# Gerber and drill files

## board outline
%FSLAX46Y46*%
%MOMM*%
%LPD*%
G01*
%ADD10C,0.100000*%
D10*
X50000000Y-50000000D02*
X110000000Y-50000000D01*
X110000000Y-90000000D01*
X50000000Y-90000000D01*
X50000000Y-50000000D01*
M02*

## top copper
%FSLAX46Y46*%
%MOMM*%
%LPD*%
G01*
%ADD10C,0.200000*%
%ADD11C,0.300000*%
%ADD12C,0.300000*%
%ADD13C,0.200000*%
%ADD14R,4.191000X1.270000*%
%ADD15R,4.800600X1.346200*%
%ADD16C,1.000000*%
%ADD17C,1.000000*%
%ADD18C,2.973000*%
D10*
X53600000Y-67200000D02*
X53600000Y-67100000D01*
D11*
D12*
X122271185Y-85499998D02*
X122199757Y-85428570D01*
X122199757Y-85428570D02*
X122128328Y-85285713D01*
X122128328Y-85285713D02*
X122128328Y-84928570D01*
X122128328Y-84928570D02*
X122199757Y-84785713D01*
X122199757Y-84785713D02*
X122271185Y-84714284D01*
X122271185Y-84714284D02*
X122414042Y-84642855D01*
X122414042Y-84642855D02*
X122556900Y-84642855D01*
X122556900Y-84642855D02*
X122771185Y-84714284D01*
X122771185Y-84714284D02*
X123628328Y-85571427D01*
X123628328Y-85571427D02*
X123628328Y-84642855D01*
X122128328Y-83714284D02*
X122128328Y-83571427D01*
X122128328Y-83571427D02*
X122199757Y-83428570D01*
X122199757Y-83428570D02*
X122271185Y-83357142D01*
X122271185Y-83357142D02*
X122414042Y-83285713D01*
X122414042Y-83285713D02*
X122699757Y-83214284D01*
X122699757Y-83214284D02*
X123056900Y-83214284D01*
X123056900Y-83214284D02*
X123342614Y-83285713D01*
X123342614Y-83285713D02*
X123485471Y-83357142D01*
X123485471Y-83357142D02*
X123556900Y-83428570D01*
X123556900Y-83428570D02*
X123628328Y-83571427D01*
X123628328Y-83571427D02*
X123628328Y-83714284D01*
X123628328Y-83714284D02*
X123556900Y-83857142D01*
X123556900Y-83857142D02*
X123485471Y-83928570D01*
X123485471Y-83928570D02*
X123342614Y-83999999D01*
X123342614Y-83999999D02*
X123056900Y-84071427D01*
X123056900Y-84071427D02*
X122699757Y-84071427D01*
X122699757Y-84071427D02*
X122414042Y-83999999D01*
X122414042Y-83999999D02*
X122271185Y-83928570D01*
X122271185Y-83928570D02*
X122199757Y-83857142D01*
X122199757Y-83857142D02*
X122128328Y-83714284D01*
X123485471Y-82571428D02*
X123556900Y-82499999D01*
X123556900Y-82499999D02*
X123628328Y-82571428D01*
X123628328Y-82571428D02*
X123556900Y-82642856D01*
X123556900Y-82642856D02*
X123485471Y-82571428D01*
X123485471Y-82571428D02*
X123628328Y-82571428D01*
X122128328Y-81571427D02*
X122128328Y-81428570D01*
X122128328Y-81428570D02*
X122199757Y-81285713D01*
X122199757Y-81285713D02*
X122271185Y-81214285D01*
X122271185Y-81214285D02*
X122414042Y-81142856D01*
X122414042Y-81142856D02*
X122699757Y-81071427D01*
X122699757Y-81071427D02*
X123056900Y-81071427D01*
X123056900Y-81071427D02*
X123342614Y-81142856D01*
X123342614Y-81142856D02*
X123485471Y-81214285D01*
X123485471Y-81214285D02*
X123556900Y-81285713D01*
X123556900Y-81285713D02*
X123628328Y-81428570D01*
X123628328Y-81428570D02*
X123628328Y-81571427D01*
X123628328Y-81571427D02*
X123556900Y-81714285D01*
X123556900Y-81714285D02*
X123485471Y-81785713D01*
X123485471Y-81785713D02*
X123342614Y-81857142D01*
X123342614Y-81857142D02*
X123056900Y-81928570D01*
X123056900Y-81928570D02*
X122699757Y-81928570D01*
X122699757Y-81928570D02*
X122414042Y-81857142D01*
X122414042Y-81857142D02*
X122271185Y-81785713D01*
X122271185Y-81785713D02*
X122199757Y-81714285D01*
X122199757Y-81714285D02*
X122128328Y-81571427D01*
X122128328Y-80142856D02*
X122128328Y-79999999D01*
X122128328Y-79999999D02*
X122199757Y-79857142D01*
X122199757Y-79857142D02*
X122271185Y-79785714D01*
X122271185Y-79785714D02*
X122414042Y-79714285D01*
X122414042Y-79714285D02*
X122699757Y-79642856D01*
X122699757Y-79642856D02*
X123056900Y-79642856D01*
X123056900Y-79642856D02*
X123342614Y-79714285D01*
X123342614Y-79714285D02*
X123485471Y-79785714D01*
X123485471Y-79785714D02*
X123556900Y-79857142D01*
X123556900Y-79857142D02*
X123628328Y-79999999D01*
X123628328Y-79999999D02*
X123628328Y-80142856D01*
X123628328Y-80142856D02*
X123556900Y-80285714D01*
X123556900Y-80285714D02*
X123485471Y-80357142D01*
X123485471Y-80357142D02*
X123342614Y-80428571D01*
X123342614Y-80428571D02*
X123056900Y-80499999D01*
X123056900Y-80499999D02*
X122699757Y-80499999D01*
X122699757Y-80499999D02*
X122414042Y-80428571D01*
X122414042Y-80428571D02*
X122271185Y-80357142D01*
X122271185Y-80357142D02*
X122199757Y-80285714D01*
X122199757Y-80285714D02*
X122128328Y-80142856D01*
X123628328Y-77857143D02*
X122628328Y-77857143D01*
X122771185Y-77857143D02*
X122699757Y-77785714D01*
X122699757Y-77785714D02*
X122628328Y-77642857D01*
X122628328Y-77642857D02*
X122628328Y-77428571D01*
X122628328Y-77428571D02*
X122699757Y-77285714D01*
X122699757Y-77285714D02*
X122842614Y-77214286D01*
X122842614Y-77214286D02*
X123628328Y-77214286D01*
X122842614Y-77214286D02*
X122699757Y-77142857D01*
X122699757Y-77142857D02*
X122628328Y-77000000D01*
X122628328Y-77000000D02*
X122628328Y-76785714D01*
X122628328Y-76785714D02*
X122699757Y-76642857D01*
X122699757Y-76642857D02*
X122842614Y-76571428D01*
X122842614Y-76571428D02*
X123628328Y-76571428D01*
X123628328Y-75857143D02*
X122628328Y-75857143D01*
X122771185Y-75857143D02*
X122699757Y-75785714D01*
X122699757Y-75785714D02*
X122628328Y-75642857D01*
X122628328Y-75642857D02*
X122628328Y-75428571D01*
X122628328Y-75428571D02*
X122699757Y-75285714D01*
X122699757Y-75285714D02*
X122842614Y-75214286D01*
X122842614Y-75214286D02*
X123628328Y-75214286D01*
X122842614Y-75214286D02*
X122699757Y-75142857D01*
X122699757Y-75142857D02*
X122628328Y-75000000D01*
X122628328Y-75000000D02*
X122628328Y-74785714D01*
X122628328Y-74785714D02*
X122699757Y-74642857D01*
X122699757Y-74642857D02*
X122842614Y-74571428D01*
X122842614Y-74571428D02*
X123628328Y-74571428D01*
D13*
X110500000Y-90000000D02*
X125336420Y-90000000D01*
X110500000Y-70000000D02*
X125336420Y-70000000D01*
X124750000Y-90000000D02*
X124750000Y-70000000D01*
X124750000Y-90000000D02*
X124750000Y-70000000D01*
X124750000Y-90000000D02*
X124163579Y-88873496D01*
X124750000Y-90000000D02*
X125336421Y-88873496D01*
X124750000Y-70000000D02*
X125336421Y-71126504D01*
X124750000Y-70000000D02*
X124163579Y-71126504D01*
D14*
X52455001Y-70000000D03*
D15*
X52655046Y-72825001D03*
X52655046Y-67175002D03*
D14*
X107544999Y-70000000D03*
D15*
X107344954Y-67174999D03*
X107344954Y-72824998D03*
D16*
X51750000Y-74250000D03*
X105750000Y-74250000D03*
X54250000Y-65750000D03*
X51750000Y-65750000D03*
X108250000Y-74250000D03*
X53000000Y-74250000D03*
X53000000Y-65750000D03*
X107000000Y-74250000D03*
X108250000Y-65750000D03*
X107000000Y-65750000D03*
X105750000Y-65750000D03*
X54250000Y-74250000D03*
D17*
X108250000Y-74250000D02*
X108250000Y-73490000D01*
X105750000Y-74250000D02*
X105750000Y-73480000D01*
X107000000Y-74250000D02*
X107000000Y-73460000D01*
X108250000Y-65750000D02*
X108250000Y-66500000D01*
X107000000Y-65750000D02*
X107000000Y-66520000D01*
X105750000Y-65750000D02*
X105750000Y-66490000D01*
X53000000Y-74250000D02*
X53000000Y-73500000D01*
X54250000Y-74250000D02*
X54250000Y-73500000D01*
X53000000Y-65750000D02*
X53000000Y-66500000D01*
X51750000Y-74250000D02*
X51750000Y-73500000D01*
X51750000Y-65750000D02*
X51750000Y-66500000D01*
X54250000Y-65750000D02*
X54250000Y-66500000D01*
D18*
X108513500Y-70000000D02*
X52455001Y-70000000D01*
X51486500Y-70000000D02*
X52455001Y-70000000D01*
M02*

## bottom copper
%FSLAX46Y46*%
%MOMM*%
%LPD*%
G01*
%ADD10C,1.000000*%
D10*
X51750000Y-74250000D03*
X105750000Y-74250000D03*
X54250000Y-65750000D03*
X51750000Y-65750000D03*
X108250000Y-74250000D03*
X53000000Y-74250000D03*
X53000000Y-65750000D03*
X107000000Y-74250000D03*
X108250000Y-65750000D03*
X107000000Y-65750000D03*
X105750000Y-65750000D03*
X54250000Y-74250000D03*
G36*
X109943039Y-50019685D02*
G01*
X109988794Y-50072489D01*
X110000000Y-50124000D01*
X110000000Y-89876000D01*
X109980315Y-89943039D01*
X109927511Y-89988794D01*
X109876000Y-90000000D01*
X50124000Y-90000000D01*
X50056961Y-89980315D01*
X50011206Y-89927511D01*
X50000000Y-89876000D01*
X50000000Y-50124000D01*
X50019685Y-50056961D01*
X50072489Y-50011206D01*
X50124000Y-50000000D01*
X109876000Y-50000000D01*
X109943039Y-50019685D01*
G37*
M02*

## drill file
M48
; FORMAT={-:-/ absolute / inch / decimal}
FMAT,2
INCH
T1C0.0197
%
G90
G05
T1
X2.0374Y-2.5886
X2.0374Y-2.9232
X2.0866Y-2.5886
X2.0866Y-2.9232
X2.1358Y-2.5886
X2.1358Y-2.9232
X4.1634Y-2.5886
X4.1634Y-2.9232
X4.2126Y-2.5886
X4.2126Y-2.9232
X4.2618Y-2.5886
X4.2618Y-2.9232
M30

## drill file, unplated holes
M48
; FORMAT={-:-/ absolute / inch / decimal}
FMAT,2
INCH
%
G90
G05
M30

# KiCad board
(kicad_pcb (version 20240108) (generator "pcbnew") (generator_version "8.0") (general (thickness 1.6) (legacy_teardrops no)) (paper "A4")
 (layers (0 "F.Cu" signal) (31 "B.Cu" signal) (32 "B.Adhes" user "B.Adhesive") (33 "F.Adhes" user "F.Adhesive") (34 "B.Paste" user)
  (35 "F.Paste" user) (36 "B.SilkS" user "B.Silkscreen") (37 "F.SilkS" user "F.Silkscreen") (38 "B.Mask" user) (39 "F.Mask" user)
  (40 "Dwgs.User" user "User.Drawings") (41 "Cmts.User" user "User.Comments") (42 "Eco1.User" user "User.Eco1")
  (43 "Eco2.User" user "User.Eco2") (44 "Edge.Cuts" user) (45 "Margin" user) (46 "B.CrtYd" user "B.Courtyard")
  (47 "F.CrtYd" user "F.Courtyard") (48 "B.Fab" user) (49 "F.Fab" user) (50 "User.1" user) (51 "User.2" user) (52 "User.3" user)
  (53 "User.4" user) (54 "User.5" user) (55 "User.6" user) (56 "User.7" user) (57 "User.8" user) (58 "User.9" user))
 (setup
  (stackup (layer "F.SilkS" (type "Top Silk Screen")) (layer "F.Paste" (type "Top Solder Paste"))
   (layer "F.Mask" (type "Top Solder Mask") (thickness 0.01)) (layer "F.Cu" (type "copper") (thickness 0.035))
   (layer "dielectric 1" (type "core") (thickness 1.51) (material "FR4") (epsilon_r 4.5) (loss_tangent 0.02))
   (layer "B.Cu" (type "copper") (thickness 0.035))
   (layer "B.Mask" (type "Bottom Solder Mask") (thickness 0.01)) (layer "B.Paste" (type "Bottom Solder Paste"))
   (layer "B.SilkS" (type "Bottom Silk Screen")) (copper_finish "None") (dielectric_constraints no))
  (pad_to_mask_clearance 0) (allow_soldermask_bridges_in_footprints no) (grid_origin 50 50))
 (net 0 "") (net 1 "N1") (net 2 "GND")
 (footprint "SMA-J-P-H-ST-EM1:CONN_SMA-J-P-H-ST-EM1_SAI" (layer "F.Cu") (at 52.16 70 90)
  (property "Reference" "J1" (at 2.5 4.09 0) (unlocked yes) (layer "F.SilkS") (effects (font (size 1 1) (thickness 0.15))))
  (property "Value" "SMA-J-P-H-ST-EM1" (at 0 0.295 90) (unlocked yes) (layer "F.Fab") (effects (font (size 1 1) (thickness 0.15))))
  (pad "1" smd rect (at 0 0.295001 90) (size 1.27 4.191) (layers "F.Cu" "F.Paste" "F.Mask") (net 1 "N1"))
  (pad "2" smd rect (at -2.825001 0.495046 90) (size 1.3462 4.8006) (layers "F.Cu" "F.Paste" "F.Mask") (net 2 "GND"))
  (pad "3" smd rect (at 2.824998 0.495046 90) (size 1.3462 4.8006) (layers "F.Cu" "F.Paste" "F.Mask") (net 2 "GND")))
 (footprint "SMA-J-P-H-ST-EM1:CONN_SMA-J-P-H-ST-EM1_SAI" (layer "F.Cu") (at 107.84 70 -90)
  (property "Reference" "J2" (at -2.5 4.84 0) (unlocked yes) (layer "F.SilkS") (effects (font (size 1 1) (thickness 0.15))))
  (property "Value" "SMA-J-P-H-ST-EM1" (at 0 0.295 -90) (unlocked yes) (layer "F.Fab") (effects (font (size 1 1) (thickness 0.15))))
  (pad "1" smd rect (at 0 0.295001 270) (size 1.27 4.191) (layers "F.Cu" "F.Paste" "F.Mask") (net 1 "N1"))
  (pad "2" smd rect (at -2.825001 0.495046 270) (size 1.3462 4.8006) (layers "F.Cu" "F.Paste" "F.Mask") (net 2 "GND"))
  (pad "3" smd rect (at 2.824998 0.495046 270) (size 1.3462 4.8006) (layers "F.Cu" "F.Paste" "F.Mask") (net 2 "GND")))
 (gr_line (start 53.6 67.2) (end 53.6 67.1) (stroke (width 0.2) (type default)) (layer "F.Cu") (net 2))
 (gr_rect (start 50 50) (end 110 90) (stroke (width 0.1) (type default)) (fill none) (layer "Edge.Cuts"))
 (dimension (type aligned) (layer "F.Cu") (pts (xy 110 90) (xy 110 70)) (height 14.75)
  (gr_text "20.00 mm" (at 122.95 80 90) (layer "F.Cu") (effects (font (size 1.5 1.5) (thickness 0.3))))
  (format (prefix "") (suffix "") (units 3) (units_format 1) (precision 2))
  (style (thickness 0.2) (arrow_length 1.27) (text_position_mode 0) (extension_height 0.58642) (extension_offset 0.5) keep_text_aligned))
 (segment (start 53 74.25) (end 53 73.5) (width 1) (layer "F.Cu") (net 2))
 (segment (start 54.25 74.25) (end 54.25 73.5) (width 1) (layer "F.Cu") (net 2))
 (segment (start 53 65.75) (end 53 66.5) (width 1) (layer "F.Cu") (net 2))
 (segment (start 105.75 65.75) (end 105.75 66.49) (width 1) (layer "F.Cu") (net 2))
 (segment (start 107 65.75) (end 107 66.52) (width 1) (layer "F.Cu") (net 2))
 (segment (start 51.75 74.25) (end 51.75 73.5) (width 1) (layer "F.Cu") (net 2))
 (segment (start 108.25 74.25) (end 108.25 73.49) (width 1) (layer "F.Cu") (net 2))
 (segment (start 51.75 65.75) (end 51.75 66.5) (width 1) (layer "F.Cu") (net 2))
 (segment (start 54.25 65.75) (end 54.25 66.5) (width 1) (layer "F.Cu") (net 2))
 (segment (start 107 74.25) (end 107 73.46) (width 1) (layer "F.Cu") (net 2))
 (segment (start 108.25 65.75) (end 108.25 66.5) (width 1) (layer "F.Cu") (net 2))
 (segment (start 105.75 74.25) (end 105.75 73.48) (width 1) (layer "F.Cu") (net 2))
 (via (at 51.75 74.25) (size 1) (drill 0.5) (layers "F.Cu" "B.Cu") (free yes) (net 2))
 (via (at 105.75 74.25) (size 1) (drill 0.5) (layers "F.Cu" "B.Cu") (free yes) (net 2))
 (via (at 54.25 65.75) (size 1) (drill 0.5) (layers "F.Cu" "B.Cu") (free yes) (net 2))
 (via (at 51.75 65.75) (size 1) (drill 0.5) (layers "F.Cu" "B.Cu") (free yes) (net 2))
 (via (at 108.25 74.25) (size 1) (drill 0.5) (layers "F.Cu" "B.Cu") (free yes) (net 2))
 (via (at 53 74.25) (size 1) (drill 0.5) (layers "F.Cu" "B.Cu") (free yes) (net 2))
 (via (at 53 65.75) (size 1) (drill 0.5) (layers "F.Cu" "B.Cu") (free yes) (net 2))
 (via (at 107 74.25) (size 1) (drill 0.5) (layers "F.Cu" "B.Cu") (free yes) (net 2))
 (via (at 108.25 65.75) (size 1) (drill 0.5) (layers "F.Cu" "B.Cu") (free yes) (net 2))
 (via (at 107 65.75) (size 1) (drill 0.5) (layers "F.Cu" "B.Cu") (free yes) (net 2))
 (via (at 105.75 65.75) (size 1) (drill 0.5) (layers "F.Cu" "B.Cu") (free yes) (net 2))
 (via (at 54.25 74.25) (size 1) (drill 0.5) (layers "F.Cu" "B.Cu") (free yes) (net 2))
 (segment (start 51.4865 70) (end 52.455001 70) (width 2.973) (layer "F.Cu") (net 1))
 (segment (start 108.5135 70) (end 52.455001 70) (width 2.973) (layer "F.Cu") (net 1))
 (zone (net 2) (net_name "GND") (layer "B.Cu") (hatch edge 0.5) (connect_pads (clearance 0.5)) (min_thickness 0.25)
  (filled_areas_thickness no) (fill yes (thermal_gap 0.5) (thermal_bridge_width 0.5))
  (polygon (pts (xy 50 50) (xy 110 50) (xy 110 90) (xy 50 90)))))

